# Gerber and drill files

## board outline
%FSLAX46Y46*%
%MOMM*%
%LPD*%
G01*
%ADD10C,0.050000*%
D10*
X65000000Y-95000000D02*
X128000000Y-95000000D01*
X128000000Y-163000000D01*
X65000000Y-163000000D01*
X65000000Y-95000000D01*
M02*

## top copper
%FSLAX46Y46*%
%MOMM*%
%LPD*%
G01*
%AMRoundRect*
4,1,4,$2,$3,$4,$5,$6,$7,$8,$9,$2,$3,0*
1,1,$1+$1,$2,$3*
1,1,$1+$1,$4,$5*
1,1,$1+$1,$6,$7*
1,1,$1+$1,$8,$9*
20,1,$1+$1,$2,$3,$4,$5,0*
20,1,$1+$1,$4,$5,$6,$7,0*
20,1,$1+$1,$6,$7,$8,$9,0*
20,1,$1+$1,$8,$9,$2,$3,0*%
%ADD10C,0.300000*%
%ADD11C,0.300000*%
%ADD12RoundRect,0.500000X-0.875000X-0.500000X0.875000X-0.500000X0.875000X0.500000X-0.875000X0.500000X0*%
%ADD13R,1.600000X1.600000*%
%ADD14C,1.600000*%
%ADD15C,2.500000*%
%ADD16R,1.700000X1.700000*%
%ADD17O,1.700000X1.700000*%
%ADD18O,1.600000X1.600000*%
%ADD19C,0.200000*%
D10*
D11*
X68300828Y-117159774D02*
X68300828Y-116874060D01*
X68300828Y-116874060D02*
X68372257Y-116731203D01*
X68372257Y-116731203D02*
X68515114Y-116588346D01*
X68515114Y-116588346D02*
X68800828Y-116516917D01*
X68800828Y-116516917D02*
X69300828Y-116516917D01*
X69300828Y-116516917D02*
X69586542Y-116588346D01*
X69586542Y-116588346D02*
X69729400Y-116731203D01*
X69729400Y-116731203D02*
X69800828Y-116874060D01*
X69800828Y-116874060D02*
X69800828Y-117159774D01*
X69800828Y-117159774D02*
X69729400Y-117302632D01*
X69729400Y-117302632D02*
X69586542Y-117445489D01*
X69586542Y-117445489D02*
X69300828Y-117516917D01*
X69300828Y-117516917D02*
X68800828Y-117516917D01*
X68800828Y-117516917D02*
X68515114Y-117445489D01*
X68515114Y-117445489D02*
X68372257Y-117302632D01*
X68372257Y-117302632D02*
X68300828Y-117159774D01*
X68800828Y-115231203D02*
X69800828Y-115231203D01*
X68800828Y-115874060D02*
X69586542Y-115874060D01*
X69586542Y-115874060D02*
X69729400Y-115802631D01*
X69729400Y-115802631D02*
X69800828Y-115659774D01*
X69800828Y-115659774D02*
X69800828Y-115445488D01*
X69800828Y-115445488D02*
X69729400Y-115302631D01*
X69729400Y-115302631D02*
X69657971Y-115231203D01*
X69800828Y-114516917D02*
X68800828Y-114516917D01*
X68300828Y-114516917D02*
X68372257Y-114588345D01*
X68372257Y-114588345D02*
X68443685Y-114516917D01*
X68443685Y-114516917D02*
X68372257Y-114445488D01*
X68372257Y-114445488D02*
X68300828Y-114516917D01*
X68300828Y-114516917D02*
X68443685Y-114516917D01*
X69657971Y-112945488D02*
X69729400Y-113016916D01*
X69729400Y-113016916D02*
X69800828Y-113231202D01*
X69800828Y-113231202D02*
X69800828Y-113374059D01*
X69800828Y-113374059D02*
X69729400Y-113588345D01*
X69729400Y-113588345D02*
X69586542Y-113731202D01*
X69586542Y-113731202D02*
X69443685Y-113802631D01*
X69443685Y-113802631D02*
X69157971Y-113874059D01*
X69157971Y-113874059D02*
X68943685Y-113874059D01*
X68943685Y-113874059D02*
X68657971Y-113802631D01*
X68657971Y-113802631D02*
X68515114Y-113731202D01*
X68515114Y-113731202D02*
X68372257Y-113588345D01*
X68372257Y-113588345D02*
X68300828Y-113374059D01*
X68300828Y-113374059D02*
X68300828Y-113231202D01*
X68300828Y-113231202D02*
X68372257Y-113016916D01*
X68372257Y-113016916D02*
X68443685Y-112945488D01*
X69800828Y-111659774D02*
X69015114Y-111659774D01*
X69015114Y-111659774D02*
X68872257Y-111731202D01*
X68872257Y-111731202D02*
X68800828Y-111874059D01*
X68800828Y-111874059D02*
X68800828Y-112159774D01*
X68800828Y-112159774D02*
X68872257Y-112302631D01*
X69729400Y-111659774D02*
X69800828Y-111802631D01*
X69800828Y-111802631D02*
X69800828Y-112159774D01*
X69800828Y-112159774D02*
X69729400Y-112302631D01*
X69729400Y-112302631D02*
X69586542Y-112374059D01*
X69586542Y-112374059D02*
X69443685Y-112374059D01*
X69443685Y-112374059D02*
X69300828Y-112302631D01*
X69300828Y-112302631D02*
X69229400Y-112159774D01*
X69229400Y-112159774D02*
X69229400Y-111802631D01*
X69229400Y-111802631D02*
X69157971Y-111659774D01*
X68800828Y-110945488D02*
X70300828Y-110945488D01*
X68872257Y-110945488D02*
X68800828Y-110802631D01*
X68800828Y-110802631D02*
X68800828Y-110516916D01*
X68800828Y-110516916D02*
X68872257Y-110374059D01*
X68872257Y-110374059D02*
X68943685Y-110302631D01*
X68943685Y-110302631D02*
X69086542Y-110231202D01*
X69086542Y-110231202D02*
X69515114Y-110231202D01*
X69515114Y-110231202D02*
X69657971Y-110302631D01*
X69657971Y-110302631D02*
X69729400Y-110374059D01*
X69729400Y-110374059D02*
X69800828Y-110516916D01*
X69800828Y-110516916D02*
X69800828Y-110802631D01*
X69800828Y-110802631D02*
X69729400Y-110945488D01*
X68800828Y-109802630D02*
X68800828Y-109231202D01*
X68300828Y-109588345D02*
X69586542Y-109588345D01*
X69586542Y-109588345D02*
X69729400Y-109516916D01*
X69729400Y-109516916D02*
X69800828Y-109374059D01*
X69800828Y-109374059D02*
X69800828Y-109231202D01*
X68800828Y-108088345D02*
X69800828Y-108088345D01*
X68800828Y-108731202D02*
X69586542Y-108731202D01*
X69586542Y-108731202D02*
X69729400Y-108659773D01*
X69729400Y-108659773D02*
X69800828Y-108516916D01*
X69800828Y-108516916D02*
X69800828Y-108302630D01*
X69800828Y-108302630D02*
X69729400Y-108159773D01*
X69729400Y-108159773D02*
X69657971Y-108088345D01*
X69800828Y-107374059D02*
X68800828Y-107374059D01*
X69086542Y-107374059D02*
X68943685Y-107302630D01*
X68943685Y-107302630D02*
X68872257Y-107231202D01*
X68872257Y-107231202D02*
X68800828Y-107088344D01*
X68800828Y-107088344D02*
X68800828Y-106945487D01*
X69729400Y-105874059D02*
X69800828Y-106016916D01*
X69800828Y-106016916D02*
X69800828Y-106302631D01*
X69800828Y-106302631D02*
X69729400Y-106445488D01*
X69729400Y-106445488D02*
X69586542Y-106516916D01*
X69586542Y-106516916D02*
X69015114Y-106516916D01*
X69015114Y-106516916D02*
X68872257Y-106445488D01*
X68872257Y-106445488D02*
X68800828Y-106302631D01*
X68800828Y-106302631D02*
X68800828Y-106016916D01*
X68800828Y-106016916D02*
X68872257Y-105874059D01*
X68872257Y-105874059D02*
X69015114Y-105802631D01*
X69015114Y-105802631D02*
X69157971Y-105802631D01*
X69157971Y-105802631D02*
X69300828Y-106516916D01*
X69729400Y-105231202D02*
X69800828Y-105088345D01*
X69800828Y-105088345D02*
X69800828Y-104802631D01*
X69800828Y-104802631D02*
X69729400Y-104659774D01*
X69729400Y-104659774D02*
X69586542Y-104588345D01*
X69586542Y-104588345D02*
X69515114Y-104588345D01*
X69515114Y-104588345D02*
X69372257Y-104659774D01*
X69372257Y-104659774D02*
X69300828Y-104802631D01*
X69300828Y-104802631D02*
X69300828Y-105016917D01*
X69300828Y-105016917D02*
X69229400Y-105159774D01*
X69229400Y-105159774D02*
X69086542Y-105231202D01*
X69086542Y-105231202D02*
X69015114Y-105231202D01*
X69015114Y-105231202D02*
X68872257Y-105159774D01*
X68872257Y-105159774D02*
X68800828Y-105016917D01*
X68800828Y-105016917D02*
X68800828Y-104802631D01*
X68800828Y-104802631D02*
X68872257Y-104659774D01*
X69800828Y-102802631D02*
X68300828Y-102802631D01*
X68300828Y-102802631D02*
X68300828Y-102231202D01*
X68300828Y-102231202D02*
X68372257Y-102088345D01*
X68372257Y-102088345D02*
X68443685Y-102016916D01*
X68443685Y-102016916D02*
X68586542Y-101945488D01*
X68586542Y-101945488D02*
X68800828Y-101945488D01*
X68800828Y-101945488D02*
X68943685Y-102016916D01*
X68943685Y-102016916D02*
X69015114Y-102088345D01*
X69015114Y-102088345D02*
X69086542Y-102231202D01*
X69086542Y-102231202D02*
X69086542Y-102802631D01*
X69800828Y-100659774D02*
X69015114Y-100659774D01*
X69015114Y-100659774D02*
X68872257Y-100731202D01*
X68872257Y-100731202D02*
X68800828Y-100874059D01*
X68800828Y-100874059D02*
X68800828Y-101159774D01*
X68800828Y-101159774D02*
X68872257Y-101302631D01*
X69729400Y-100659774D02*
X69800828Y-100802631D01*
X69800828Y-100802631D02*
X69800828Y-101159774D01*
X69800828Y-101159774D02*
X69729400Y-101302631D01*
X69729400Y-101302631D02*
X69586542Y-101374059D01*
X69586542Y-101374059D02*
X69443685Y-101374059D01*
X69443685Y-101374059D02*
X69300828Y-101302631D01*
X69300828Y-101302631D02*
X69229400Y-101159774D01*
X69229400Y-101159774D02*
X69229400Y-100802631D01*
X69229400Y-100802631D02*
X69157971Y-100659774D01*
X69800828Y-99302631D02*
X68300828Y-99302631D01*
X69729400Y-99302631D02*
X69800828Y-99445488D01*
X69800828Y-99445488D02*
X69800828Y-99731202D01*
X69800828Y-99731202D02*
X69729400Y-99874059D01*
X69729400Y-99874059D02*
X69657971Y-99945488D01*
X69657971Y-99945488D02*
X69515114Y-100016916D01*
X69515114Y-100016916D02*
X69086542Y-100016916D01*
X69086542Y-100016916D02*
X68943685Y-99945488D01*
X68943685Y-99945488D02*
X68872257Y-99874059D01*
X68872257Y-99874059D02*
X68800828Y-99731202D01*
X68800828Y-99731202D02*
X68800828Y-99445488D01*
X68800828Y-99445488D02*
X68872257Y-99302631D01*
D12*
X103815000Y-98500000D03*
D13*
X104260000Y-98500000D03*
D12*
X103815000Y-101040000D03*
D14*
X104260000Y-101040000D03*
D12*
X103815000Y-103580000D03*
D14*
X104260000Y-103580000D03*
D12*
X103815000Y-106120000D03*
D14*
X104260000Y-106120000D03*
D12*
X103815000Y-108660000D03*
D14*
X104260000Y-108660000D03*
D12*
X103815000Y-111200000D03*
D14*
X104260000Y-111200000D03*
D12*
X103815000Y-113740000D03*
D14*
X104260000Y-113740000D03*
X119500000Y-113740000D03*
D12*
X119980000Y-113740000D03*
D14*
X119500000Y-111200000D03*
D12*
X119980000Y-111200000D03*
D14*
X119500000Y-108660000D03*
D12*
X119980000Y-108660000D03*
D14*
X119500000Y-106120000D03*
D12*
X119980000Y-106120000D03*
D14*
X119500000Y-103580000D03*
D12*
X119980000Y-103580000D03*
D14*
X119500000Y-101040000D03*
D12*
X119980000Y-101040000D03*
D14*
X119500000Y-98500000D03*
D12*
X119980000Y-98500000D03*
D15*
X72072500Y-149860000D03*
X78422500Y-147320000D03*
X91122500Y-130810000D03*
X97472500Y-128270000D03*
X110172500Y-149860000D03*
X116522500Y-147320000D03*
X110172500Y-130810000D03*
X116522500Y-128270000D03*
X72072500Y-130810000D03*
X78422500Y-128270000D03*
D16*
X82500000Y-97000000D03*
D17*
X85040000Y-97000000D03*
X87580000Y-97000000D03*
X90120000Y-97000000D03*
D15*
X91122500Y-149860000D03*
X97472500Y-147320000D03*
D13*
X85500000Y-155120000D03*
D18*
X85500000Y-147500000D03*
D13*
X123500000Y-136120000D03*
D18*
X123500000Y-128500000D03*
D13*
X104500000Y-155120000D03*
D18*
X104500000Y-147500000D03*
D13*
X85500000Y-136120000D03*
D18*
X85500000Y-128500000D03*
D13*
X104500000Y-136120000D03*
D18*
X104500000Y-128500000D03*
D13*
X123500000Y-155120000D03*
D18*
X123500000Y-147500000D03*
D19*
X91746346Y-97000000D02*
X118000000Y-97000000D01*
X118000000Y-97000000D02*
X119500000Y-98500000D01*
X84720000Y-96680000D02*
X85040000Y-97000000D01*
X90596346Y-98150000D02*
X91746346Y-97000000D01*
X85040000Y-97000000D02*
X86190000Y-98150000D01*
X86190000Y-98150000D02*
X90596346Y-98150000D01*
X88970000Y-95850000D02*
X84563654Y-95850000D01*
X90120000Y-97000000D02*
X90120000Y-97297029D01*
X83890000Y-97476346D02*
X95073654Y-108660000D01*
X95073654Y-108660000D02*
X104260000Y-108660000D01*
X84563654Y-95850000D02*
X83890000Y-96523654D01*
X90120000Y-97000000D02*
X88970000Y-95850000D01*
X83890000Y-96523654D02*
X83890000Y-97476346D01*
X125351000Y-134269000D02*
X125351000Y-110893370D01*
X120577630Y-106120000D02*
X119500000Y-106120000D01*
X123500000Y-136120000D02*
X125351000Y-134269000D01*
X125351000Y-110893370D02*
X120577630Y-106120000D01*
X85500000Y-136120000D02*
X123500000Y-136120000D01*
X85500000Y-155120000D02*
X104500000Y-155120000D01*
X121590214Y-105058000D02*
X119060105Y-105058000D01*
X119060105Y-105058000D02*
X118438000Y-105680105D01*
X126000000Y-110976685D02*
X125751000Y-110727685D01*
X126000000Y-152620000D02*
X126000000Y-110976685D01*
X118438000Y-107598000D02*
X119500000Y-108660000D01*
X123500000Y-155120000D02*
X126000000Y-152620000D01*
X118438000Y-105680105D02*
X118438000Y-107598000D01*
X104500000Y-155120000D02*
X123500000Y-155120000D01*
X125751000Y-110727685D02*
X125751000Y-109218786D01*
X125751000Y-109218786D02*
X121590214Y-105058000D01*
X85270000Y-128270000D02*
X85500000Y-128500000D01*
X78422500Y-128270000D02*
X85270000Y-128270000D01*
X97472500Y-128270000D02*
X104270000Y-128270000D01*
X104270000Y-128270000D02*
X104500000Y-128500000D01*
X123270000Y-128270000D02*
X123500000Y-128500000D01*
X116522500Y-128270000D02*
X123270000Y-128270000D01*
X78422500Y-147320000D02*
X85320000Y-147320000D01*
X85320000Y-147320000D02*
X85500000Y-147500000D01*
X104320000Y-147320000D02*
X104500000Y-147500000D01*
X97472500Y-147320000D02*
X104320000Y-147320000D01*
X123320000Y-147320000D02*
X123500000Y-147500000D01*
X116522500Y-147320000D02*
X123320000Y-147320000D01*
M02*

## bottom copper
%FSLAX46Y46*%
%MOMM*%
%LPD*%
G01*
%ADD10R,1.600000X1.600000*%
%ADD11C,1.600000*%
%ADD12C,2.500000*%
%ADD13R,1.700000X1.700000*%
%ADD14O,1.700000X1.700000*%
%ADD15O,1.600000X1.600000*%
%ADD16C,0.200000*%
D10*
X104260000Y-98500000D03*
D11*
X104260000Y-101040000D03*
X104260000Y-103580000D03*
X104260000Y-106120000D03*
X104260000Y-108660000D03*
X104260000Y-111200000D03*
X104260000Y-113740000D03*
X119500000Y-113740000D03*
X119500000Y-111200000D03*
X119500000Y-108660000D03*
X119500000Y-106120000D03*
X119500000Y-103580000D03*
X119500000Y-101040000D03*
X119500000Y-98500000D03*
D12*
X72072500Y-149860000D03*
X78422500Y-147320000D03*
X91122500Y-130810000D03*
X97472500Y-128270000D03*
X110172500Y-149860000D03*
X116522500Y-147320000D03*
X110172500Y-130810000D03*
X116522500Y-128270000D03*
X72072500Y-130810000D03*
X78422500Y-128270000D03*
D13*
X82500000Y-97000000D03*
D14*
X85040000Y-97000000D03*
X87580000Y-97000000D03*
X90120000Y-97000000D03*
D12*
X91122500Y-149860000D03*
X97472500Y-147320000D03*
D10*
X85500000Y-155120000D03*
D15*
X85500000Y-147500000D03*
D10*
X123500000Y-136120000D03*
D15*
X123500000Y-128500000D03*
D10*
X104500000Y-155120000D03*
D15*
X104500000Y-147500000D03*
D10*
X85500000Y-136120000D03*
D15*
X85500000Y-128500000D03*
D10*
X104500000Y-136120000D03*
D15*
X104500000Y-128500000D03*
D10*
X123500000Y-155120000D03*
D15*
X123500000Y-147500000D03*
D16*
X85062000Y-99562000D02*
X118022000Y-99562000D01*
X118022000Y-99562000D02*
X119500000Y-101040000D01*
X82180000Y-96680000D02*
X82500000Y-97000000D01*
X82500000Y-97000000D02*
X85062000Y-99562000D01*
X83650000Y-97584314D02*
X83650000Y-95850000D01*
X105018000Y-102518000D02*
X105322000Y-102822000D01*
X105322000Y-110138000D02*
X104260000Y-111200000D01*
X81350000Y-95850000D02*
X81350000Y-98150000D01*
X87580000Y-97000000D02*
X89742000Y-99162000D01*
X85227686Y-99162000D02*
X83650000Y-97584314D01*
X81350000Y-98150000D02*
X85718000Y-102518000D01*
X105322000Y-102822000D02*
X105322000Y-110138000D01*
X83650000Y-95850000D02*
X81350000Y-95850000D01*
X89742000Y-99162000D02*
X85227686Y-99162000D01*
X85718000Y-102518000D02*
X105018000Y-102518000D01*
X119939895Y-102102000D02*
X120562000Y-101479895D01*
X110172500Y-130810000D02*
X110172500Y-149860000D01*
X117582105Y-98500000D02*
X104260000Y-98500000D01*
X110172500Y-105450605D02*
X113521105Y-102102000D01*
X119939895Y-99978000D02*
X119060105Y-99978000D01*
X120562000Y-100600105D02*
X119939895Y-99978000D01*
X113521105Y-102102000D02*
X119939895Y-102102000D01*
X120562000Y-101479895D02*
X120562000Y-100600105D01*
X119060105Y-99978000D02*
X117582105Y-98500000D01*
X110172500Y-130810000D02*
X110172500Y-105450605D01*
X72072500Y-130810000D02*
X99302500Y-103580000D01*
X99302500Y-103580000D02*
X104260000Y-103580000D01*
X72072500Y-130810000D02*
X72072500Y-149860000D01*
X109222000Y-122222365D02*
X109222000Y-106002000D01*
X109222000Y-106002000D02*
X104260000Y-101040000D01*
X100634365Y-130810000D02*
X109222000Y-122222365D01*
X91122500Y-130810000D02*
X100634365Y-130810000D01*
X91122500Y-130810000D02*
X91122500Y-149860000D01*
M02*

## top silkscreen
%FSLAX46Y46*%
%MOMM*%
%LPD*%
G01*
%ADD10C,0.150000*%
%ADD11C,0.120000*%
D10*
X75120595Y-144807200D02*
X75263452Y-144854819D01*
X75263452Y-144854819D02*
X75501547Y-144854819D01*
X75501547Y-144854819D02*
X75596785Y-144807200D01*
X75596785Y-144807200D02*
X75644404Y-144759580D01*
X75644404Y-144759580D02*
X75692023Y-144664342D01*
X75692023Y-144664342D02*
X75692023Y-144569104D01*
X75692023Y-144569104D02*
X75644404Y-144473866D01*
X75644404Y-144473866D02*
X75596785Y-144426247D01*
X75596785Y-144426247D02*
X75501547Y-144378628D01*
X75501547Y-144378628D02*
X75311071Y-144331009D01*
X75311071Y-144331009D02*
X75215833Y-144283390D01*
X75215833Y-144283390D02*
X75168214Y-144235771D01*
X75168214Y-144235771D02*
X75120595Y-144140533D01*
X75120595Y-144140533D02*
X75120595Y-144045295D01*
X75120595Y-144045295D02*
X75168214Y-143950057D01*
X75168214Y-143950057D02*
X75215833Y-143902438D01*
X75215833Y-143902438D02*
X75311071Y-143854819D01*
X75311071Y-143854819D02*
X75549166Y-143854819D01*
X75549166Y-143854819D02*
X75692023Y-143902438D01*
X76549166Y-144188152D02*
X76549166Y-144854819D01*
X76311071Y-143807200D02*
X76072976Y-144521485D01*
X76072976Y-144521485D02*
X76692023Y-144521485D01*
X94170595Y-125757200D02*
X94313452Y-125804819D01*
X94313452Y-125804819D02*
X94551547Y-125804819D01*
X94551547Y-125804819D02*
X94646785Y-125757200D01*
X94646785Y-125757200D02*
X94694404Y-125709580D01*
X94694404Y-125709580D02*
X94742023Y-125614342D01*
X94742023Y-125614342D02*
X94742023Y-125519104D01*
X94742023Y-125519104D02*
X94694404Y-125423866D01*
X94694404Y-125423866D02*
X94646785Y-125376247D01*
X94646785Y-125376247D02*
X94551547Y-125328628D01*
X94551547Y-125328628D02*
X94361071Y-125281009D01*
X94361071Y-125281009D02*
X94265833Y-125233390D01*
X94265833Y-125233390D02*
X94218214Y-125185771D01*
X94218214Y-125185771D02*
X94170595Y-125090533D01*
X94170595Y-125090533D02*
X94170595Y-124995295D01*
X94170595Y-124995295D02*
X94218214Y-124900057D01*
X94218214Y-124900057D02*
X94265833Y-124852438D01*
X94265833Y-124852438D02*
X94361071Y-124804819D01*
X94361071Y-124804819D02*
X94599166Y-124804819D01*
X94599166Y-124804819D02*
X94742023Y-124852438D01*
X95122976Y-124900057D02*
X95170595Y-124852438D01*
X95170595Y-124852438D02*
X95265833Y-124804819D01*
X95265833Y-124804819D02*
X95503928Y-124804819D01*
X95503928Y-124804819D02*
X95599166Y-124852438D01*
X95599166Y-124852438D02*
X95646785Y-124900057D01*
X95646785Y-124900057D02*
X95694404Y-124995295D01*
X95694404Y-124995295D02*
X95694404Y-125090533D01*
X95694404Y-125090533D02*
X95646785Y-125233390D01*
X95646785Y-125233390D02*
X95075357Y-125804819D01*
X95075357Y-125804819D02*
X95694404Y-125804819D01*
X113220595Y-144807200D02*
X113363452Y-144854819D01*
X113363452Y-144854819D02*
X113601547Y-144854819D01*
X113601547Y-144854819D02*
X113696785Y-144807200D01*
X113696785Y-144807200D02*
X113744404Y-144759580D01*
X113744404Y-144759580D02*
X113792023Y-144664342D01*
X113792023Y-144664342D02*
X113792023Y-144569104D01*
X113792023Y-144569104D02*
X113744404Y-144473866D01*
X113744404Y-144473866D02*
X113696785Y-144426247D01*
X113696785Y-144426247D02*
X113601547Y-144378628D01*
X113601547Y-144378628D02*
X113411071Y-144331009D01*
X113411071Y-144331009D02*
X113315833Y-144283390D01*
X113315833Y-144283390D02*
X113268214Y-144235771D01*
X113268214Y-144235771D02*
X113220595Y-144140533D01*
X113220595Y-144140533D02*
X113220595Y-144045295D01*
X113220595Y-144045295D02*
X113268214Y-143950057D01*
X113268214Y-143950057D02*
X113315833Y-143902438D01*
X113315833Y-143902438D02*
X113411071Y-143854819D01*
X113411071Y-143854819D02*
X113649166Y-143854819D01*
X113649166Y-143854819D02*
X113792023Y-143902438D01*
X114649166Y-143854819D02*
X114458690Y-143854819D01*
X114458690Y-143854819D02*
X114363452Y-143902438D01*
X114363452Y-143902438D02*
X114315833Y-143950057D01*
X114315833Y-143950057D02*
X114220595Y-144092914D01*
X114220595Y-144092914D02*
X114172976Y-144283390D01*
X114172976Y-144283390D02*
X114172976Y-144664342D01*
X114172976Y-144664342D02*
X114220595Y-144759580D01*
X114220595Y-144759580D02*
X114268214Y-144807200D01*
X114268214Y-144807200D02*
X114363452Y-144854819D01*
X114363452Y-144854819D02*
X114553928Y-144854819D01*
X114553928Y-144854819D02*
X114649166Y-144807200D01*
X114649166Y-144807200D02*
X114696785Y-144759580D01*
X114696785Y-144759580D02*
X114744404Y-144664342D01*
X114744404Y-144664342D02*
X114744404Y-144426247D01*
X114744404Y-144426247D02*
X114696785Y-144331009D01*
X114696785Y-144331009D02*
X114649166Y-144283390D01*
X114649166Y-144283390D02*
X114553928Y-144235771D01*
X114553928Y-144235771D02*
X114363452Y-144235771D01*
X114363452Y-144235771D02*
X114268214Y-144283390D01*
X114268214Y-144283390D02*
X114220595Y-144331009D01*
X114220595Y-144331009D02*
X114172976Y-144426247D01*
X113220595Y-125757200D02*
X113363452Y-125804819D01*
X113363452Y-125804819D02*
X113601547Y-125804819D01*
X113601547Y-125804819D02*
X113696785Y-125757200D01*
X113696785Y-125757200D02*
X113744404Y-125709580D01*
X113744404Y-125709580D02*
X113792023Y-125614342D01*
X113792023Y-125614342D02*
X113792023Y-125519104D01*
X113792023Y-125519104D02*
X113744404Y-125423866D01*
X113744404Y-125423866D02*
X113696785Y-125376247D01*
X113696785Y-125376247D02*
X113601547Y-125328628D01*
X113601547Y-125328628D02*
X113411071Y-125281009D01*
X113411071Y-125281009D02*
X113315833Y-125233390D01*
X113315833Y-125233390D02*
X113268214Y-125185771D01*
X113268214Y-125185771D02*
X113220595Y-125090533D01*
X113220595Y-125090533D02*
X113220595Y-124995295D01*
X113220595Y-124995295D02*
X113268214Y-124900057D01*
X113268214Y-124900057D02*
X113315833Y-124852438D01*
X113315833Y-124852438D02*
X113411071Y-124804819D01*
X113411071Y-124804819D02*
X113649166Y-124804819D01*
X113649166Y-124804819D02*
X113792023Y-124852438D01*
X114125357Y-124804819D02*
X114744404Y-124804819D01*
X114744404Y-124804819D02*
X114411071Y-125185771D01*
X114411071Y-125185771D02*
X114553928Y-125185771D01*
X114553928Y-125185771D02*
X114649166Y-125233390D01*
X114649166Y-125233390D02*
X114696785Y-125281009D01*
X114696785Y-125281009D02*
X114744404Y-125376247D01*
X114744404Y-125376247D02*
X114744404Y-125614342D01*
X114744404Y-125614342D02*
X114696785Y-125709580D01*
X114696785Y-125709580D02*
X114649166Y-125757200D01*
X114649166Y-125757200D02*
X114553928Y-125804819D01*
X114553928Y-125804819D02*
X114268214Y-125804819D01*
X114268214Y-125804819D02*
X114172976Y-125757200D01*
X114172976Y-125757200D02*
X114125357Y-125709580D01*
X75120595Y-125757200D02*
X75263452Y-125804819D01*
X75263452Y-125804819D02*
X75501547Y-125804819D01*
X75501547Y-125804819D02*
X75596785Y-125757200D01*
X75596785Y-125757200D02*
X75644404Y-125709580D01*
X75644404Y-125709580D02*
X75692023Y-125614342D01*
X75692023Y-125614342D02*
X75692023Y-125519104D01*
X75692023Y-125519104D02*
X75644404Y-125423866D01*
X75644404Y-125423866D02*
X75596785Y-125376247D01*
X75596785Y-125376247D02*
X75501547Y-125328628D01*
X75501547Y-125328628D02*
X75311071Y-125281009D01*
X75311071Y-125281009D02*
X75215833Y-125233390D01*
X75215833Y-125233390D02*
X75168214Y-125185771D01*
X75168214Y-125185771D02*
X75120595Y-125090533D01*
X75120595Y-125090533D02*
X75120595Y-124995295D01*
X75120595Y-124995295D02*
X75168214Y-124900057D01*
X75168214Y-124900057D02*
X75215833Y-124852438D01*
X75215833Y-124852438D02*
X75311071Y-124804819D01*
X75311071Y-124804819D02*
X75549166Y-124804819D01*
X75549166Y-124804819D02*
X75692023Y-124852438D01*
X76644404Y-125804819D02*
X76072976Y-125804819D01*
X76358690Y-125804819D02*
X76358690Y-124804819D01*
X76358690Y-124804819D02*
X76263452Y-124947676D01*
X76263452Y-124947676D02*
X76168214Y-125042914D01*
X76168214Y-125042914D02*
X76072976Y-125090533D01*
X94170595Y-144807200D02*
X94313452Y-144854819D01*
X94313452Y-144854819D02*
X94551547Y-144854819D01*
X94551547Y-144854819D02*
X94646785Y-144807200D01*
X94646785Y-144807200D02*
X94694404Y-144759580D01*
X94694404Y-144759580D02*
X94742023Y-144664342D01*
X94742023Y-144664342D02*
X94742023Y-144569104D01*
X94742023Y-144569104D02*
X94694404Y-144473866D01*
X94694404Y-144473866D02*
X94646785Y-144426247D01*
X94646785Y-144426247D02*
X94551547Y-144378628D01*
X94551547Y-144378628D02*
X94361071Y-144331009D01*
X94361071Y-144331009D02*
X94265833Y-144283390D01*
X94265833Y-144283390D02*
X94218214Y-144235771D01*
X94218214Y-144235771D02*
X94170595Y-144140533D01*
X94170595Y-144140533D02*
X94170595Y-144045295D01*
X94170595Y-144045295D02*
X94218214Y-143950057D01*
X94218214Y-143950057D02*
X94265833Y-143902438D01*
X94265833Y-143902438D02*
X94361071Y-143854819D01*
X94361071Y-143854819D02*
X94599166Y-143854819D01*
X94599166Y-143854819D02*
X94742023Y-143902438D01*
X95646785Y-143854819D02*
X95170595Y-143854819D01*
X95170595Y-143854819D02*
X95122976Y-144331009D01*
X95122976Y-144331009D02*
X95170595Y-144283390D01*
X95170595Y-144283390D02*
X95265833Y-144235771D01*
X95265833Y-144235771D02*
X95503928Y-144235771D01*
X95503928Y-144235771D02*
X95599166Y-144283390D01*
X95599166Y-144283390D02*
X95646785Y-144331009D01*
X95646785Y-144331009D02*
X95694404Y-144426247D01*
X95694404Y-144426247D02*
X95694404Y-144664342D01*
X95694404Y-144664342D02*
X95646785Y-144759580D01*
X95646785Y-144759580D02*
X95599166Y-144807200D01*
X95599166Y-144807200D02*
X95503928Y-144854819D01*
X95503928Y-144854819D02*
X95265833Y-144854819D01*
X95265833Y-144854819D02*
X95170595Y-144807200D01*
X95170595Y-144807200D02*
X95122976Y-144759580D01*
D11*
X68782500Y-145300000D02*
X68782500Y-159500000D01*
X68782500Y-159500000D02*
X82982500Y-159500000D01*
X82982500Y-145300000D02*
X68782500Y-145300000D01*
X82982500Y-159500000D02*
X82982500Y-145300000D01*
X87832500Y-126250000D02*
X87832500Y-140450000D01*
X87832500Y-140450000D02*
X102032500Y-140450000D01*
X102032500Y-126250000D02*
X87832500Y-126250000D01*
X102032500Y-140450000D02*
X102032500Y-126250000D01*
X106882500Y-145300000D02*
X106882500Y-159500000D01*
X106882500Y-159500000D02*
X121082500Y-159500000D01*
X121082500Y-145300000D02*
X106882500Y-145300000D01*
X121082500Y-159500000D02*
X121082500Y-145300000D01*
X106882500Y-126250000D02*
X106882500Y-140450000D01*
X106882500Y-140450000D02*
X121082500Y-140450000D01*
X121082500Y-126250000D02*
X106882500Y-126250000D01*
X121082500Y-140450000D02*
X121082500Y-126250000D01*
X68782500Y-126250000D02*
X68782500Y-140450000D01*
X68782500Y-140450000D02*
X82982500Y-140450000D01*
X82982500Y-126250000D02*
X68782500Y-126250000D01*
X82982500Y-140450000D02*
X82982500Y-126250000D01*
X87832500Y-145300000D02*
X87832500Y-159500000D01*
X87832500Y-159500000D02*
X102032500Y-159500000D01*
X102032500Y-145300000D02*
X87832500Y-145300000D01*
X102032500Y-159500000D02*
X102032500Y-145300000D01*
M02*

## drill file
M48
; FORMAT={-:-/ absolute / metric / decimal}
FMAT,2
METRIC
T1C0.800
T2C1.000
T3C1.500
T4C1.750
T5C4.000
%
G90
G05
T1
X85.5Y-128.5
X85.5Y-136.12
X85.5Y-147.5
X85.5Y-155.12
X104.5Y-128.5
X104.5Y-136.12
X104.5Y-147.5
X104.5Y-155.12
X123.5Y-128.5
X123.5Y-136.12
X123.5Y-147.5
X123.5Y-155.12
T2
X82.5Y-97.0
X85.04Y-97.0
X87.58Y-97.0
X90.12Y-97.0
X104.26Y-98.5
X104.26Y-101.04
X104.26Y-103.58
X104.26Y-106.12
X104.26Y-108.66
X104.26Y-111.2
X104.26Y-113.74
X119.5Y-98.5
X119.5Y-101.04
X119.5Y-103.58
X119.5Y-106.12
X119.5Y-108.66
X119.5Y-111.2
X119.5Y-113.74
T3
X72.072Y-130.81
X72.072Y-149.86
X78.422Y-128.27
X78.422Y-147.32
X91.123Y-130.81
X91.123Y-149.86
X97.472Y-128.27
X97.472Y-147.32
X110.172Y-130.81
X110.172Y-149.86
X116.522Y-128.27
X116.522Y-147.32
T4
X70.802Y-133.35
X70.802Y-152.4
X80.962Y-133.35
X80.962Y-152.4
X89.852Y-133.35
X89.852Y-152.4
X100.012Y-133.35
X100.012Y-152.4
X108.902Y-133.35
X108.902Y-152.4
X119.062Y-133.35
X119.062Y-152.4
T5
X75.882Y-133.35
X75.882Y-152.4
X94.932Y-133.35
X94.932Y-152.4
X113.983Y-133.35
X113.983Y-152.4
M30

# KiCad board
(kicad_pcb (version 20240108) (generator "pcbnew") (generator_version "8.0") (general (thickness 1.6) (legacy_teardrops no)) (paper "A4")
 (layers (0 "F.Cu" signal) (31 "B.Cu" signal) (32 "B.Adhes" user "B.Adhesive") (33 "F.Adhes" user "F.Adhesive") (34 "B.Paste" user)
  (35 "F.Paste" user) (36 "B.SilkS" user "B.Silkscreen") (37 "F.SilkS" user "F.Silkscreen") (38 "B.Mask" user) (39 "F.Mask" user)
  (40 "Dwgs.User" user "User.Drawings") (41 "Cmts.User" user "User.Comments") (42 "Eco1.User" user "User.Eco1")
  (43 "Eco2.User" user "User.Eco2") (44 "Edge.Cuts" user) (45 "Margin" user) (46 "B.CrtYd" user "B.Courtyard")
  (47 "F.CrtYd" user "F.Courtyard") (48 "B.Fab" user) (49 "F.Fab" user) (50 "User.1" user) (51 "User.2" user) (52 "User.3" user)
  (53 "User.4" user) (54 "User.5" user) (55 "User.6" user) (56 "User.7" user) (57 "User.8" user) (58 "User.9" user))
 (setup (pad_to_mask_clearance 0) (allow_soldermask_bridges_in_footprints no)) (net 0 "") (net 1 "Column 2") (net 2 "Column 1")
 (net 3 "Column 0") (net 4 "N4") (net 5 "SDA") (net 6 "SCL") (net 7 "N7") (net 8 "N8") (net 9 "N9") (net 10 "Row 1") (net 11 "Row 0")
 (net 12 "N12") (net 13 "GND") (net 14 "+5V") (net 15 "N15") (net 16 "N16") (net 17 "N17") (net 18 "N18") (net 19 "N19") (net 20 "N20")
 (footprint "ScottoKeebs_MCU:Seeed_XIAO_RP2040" (layer "F.Cu") (at 111.88 106.12)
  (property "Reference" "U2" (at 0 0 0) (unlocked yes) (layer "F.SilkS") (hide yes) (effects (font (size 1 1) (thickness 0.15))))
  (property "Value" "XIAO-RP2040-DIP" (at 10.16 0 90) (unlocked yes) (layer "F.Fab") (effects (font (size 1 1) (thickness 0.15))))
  (pad "1" smd roundrect (at -8.065 -7.62) (size 2.75 2) (layers "F.Cu" "F.Paste" "F.Mask") (roundrect_rratio 0.25) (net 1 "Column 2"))
  (pad "1" thru_hole rect (at -7.62 -7.62 90) (size 1.6 1.6) (drill 1) (layers "*.Cu" "*.Mask") (remove_unused_layers no) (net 1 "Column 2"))
  (pad "2" smd roundrect (at -8.065 -5.08) (size 2.75 2) (layers "F.Cu" "F.Paste" "F.Mask") (roundrect_rratio 0.25) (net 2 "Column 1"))
  (pad "2" thru_hole circle (at -7.62 -5.08 90) (size 1.6 1.6) (drill 1) (layers "*.Cu" "*.Mask") (remove_unused_layers no)
   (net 2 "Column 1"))
  (pad "3" smd roundrect (at -8.065 -2.54) (size 2.75 2) (layers "F.Cu" "F.Paste" "F.Mask") (roundrect_rratio 0.25) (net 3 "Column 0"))
  (pad "3" thru_hole circle (at -7.62 -2.54 90) (size 1.6 1.6) (drill 1) (layers "*.Cu" "*.Mask") (remove_unused_layers no)
   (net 3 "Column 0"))
  (pad "4" smd roundrect (at -8.065 0) (size 2.75 2) (layers "F.Cu" "F.Paste" "F.Mask") (roundrect_rratio 0.25) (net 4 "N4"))
  (pad "4" thru_hole circle (at -7.62 0 90) (size 1.6 1.6) (drill 1) (layers "*.Cu" "*.Mask") (remove_unused_layers no) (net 4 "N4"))
  (pad "5" smd roundrect (at -8.065 2.54) (size 2.75 2) (layers "F.Cu" "F.Paste" "F.Mask") (roundrect_rratio 0.25) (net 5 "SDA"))
  (pad "5" thru_hole circle (at -7.62 2.54 90) (size 1.6 1.6) (drill 1) (layers "*.Cu" "*.Mask") (remove_unused_layers no) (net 5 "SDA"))
  (pad "6" smd roundrect (at -8.065 5.08) (size 2.75 2) (layers "F.Cu" "F.Paste" "F.Mask") (roundrect_rratio 0.25) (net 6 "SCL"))
  (pad "6" thru_hole circle (at -7.62 5.08 90) (size 1.6 1.6) (drill 1) (layers "*.Cu" "*.Mask") (remove_unused_layers no) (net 6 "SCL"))
  (pad "7" smd roundrect (at -8.065 7.62) (size 2.75 2) (layers "F.Cu" "F.Paste" "F.Mask") (roundrect_rratio 0.25) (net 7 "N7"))
  (pad "7" thru_hole circle (at -7.62 7.62 90) (size 1.6 1.6) (drill 1) (layers "*.Cu" "*.Mask") (remove_unused_layers no) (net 7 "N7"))
  (pad "8" thru_hole circle (at 7.62 7.62 90) (size 1.6 1.6) (drill 1) (layers "*.Cu" "*.Mask") (remove_unused_layers no) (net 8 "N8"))
  (pad "8" smd roundrect (at 8.1 7.62) (size 2.75 2) (layers "F.Cu" "F.Paste" "F.Mask") (roundrect_rratio 0.25) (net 8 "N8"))
  (pad "9" thru_hole circle (at 7.62 5.08 90) (size 1.6 1.6) (drill 1) (layers "*.Cu" "*.Mask") (remove_unused_layers no) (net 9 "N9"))
  (pad "9" smd roundrect (at 8.1 5.08) (size 2.75 2) (layers "F.Cu" "F.Paste" "F.Mask") (roundrect_rratio 0.25) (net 9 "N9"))
  (pad "10" thru_hole circle (at 7.62 2.54 90) (size 1.6 1.6) (drill 1) (layers "*.Cu" "*.Mask") (remove_unused_layers no) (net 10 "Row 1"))
  (pad "10" smd roundrect (at 8.1 2.54) (size 2.75 2) (layers "F.Cu" "F.Paste" "F.Mask") (roundrect_rratio 0.25) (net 10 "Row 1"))
  (pad "11" thru_hole circle (at 7.62 0 90) (size 1.6 1.6) (drill 1) (layers "*.Cu" "*.Mask") (remove_unused_layers no) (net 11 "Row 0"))
  (pad "11" smd roundrect (at 8.1 0) (size 2.75 2) (layers "F.Cu" "F.Paste" "F.Mask") (roundrect_rratio 0.25) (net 11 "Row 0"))
  (pad "12" thru_hole circle (at 7.62 -2.54 90) (size 1.6 1.6) (drill 1) (layers "*.Cu" "*.Mask") (remove_unused_layers no) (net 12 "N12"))
  (pad "12" smd roundrect (at 8.1 -2.54) (size 2.75 2) (layers "F.Cu" "F.Paste" "F.Mask") (roundrect_rratio 0.25) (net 12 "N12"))
  (pad "13" thru_hole circle (at 7.62 -5.08 90) (size 1.6 1.6) (drill 1) (layers "*.Cu" "*.Mask") (remove_unused_layers no) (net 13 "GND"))
  (pad "13" smd roundrect (at 8.1 -5.08) (size 2.75 2) (layers "F.Cu" "F.Paste" "F.Mask") (roundrect_rratio 0.25) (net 13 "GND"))
  (pad "14" thru_hole circle (at 7.62 -7.62 90) (size 1.6 1.6) (drill 1) (layers "*.Cu" "*.Mask") (remove_unused_layers no) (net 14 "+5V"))
  (pad "14" smd roundrect (at 8.1 -7.62) (size 2.75 2) (layers "F.Cu" "F.Paste" "F.Mask") (roundrect_rratio 0.25) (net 14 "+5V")))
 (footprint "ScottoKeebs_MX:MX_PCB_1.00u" (layer "F.Cu") (at 75.8825 152.4)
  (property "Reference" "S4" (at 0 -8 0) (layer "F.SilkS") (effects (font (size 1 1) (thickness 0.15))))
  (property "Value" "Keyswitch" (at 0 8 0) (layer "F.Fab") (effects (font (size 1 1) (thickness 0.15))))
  (fp_line (start -7.1 -7.1) (end -7.1 7.1) (stroke (width 0.12) (type solid)) (layer "F.SilkS"))
  (fp_line (start -7.1 7.1) (end 7.1 7.1) (stroke (width 0.12) (type solid)) (layer "F.SilkS"))
  (fp_line (start 7.1 -7.1) (end -7.1 -7.1) (stroke (width 0.12) (type solid)) (layer "F.SilkS"))
  (fp_line (start 7.1 7.1) (end 7.1 -7.1) (stroke (width 0.12) (type solid)) (layer "F.SilkS"))
  (pad "" np_thru_hole circle (at -5.08 0) (size 1.75 1.75) (drill 1.75) (layers "*.Cu" "*.Mask"))
  (pad "" np_thru_hole circle (at 0 0) (size 4 4) (drill 4) (layers "*.Cu" "*.Mask"))
  (pad "" np_thru_hole circle (at 5.08 0) (size 1.75 1.75) (drill 1.75) (layers "*.Cu" "*.Mask"))
  (pad "1" thru_hole circle (at -3.81 -2.54) (size 2.5 2.5) (drill 1.5) (layers "*.Cu" "*.Mask") (remove_unused_layers no)
   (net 3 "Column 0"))
  (pad "2" thru_hole circle (at 2.54 -5.08) (size 2.5 2.5) (drill 1.5) (layers "*.Cu" "*.Mask") (remove_unused_layers no) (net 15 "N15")))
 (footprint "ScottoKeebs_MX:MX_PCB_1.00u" (layer "F.Cu") (at 94.9325 133.35)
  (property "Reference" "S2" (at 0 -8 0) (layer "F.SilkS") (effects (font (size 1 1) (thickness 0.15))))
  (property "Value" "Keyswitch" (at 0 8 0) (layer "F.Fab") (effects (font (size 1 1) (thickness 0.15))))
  (fp_line (start -7.1 -7.1) (end -7.1 7.1) (stroke (width 0.12) (type solid)) (layer "F.SilkS"))
  (fp_line (start -7.1 7.1) (end 7.1 7.1) (stroke (width 0.12) (type solid)) (layer "F.SilkS"))
  (fp_line (start 7.1 -7.1) (end -7.1 -7.1) (stroke (width 0.12) (type solid)) (layer "F.SilkS"))
  (fp_line (start 7.1 7.1) (end 7.1 -7.1) (stroke (width 0.12) (type solid)) (layer "F.SilkS"))
  (pad "" np_thru_hole circle (at -5.08 0) (size 1.75 1.75) (drill 1.75) (layers "*.Cu" "*.Mask"))
  (pad "" np_thru_hole circle (at 0 0) (size 4 4) (drill 4) (layers "*.Cu" "*.Mask"))
  (pad "" np_thru_hole circle (at 5.08 0) (size 1.75 1.75) (drill 1.75) (layers "*.Cu" "*.Mask"))
  (pad "1" thru_hole circle (at -3.81 -2.54) (size 2.5 2.5) (drill 1.5) (layers "*.Cu" "*.Mask") (remove_unused_layers no)
   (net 2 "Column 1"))
  (pad "2" thru_hole circle (at 2.54 -5.08) (size 2.5 2.5) (drill 1.5) (layers "*.Cu" "*.Mask") (remove_unused_layers no) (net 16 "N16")))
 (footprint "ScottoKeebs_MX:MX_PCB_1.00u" (layer "F.Cu") (at 113.9825 152.4)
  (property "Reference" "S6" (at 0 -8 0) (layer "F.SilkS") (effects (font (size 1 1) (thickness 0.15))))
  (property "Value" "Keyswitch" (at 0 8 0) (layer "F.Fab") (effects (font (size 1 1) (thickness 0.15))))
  (fp_line (start -7.1 -7.1) (end -7.1 7.1) (stroke (width 0.12) (type solid)) (layer "F.SilkS"))
  (fp_line (start -7.1 7.1) (end 7.1 7.1) (stroke (width 0.12) (type solid)) (layer "F.SilkS"))
  (fp_line (start 7.1 -7.1) (end -7.1 -7.1) (stroke (width 0.12) (type solid)) (layer "F.SilkS"))
  (fp_line (start 7.1 7.1) (end 7.1 -7.1) (stroke (width 0.12) (type solid)) (layer "F.SilkS"))
  (pad "" np_thru_hole circle (at -5.08 0) (size 1.75 1.75) (drill 1.75) (layers "*.Cu" "*.Mask"))
  (pad "" np_thru_hole circle (at 0 0) (size 4 4) (drill 4) (layers "*.Cu" "*.Mask"))
  (pad "" np_thru_hole circle (at 5.08 0) (size 1.75 1.75) (drill 1.75) (layers "*.Cu" "*.Mask"))
  (pad "1" thru_hole circle (at -3.81 -2.54) (size 2.5 2.5) (drill 1.5) (layers "*.Cu" "*.Mask") (remove_unused_layers no)
   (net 1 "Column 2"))
  (pad "2" thru_hole circle (at 2.54 -5.08) (size 2.5 2.5) (drill 1.5) (layers "*.Cu" "*.Mask") (remove_unused_layers no) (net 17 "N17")))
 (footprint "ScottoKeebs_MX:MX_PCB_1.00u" (layer "F.Cu") (at 113.9825 133.35)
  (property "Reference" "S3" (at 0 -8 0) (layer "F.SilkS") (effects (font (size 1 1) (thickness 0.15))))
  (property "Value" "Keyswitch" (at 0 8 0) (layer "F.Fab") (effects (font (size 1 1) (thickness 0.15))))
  (fp_line (start -7.1 -7.1) (end -7.1 7.1) (stroke (width 0.12) (type solid)) (layer "F.SilkS"))
  (fp_line (start -7.1 7.1) (end 7.1 7.1) (stroke (width 0.12) (type solid)) (layer "F.SilkS"))
  (fp_line (start 7.1 -7.1) (end -7.1 -7.1) (stroke (width 0.12) (type solid)) (layer "F.SilkS"))
  (fp_line (start 7.1 7.1) (end 7.1 -7.1) (stroke (width 0.12) (type solid)) (layer "F.SilkS"))
  (pad "" np_thru_hole circle (at -5.08 0) (size 1.75 1.75) (drill 1.75) (layers "*.Cu" "*.Mask"))
  (pad "" np_thru_hole circle (at 0 0) (size 4 4) (drill 4) (layers "*.Cu" "*.Mask"))
  (pad "" np_thru_hole circle (at 5.08 0) (size 1.75 1.75) (drill 1.75) (layers "*.Cu" "*.Mask"))
  (pad "1" thru_hole circle (at -3.81 -2.54) (size 2.5 2.5) (drill 1.5) (layers "*.Cu" "*.Mask") (remove_unused_layers no)
   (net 1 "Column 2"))
  (pad "2" thru_hole circle (at 2.54 -5.08) (size 2.5 2.5) (drill 1.5) (layers "*.Cu" "*.Mask") (remove_unused_layers no) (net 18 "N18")))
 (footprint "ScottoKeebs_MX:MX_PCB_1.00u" (layer "F.Cu") (at 75.8825 133.35)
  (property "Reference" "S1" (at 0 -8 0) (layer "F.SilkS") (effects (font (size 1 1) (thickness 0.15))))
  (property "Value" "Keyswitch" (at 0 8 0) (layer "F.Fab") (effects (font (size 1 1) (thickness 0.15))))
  (fp_line (start -7.1 -7.1) (end -7.1 7.1) (stroke (width 0.12) (type solid)) (layer "F.SilkS"))
  (fp_line (start -7.1 7.1) (end 7.1 7.1) (stroke (width 0.12) (type solid)) (layer "F.SilkS"))
  (fp_line (start 7.1 -7.1) (end -7.1 -7.1) (stroke (width 0.12) (type solid)) (layer "F.SilkS"))
  (fp_line (start 7.1 7.1) (end 7.1 -7.1) (stroke (width 0.12) (type solid)) (layer "F.SilkS"))
  (pad "" np_thru_hole circle (at -5.08 0) (size 1.75 1.75) (drill 1.75) (layers "*.Cu" "*.Mask"))
  (pad "" np_thru_hole circle (at 0 0) (size 4 4) (drill 4) (layers "*.Cu" "*.Mask"))
  (pad "" np_thru_hole circle (at 5.08 0) (size 1.75 1.75) (drill 1.75) (layers "*.Cu" "*.Mask"))
  (pad "1" thru_hole circle (at -3.81 -2.54) (size 2.5 2.5) (drill 1.5) (layers "*.Cu" "*.Mask") (remove_unused_layers no)
   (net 3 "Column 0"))
  (pad "2" thru_hole circle (at 2.54 -5.08) (size 2.5 2.5) (drill 1.5) (layers "*.Cu" "*.Mask") (remove_unused_layers no) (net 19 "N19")))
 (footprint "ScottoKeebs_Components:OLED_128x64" (layer "F.Cu") (at 86.31 97)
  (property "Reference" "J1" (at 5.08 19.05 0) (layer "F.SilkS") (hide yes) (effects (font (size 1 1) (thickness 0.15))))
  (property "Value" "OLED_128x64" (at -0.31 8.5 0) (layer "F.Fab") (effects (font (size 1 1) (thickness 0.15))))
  (pad "1" thru_hole rect (at -3.81 0 90) (size 1.7 1.7) (drill 1) (layers "*.Cu" "*.Mask") (remove_unused_layers no) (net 13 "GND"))
  (pad "2" thru_hole oval (at -1.27 0 90) (size 1.7 1.7) (drill 1) (layers "*.Cu" "*.Mask") (remove_unused_layers no) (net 14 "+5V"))
  (pad "3" thru_hole oval (at 1.27 0 90) (size 1.7 1.7) (drill 1) (layers "*.Cu" "*.Mask") (remove_unused_layers no) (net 6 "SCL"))
  (pad "4" thru_hole oval (at 3.81 0 90) (size 1.7 1.7) (drill 1) (layers "*.Cu" "*.Mask") (remove_unused_layers no) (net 5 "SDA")))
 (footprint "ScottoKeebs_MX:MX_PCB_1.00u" (layer "F.Cu") (at 94.9325 152.4)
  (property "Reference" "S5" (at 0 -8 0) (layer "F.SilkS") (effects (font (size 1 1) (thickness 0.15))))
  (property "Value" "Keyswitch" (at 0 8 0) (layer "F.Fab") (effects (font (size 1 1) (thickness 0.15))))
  (fp_line (start -7.1 -7.1) (end -7.1 7.1) (stroke (width 0.12) (type solid)) (layer "F.SilkS"))
  (fp_line (start -7.1 7.1) (end 7.1 7.1) (stroke (width 0.12) (type solid)) (layer "F.SilkS"))
  (fp_line (start 7.1 -7.1) (end -7.1 -7.1) (stroke (width 0.12) (type solid)) (layer "F.SilkS"))
  (fp_line (start 7.1 7.1) (end 7.1 -7.1) (stroke (width 0.12) (type solid)) (layer "F.SilkS"))
  (pad "" np_thru_hole circle (at -5.08 0) (size 1.75 1.75) (drill 1.75) (layers "*.Cu" "*.Mask"))
  (pad "" np_thru_hole circle (at 0 0) (size 4 4) (drill 4) (layers "*.Cu" "*.Mask"))
  (pad "" np_thru_hole circle (at 5.08 0) (size 1.75 1.75) (drill 1.75) (layers "*.Cu" "*.Mask"))
  (pad "1" thru_hole circle (at -3.81 -2.54) (size 2.5 2.5) (drill 1.5) (layers "*.Cu" "*.Mask") (remove_unused_layers no)
   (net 2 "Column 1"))
  (pad "2" thru_hole circle (at 2.54 -5.08) (size 2.5 2.5) (drill 1.5) (layers "*.Cu" "*.Mask") (remove_unused_layers no) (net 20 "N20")))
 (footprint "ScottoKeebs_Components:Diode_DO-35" (layer "B.Cu") (at 85.5 155.12 90)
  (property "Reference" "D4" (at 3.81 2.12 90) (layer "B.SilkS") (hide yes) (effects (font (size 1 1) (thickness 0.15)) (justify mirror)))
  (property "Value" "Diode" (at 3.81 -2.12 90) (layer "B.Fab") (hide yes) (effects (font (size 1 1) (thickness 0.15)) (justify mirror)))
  (pad "1" thru_hole rect (at 0 0 90) (size 1.6 1.6) (drill 0.8) (layers "*.Cu" "*.Mask") (remove_unused_layers no) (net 10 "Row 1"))
  (pad "2" thru_hole oval (at 7.62 0 90) (size 1.6 1.6) (drill 0.8) (layers "*.Cu" "*.Mask") (remove_unused_layers no) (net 15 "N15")))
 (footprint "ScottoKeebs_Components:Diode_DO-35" (layer "B.Cu") (at 123.5 136.12 90)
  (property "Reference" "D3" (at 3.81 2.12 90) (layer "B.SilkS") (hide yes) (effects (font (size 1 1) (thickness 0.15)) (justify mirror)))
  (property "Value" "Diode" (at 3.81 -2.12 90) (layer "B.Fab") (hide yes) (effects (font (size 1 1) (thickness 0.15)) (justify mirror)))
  (pad "1" thru_hole rect (at 0 0 90) (size 1.6 1.6) (drill 0.8) (layers "*.Cu" "*.Mask") (remove_unused_layers no) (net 11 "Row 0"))
  (pad "2" thru_hole oval (at 7.62 0 90) (size 1.6 1.6) (drill 0.8) (layers "*.Cu" "*.Mask") (remove_unused_layers no) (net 18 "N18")))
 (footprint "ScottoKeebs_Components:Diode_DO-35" (layer "B.Cu") (at 104.5 155.12 90)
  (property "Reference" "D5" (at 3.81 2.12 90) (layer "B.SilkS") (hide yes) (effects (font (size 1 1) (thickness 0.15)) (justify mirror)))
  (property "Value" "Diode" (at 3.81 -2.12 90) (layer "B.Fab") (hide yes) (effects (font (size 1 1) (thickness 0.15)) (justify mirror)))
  (pad "1" thru_hole rect (at 0 0 90) (size 1.6 1.6) (drill 0.8) (layers "*.Cu" "*.Mask") (remove_unused_layers no) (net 10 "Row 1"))
  (pad "2" thru_hole oval (at 7.62 0 90) (size 1.6 1.6) (drill 0.8) (layers "*.Cu" "*.Mask") (remove_unused_layers no) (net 20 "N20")))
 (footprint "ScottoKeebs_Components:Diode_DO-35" (layer "B.Cu") (at 85.5 136.12 90)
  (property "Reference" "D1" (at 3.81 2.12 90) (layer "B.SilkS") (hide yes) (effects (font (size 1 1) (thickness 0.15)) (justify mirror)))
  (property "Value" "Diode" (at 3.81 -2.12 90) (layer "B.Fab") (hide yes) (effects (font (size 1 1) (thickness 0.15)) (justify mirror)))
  (pad "1" thru_hole rect (at 0 0 90) (size 1.6 1.6) (drill 0.8) (layers "*.Cu" "*.Mask") (remove_unused_layers no) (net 11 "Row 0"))
  (pad "2" thru_hole oval (at 7.62 0 90) (size 1.6 1.6) (drill 0.8) (layers "*.Cu" "*.Mask") (remove_unused_layers no) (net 19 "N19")))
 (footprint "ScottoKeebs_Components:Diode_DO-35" (layer "B.Cu") (at 104.5 136.12 90)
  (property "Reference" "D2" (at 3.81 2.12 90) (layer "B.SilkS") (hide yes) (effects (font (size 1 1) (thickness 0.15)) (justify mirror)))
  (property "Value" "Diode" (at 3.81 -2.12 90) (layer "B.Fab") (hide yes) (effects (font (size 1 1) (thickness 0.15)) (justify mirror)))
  (pad "1" thru_hole rect (at 0 0 90) (size 1.6 1.6) (drill 0.8) (layers "*.Cu" "*.Mask") (remove_unused_layers no) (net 11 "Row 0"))
  (pad "2" thru_hole oval (at 7.62 0 90) (size 1.6 1.6) (drill 0.8) (layers "*.Cu" "*.Mask") (remove_unused_layers no) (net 16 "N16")))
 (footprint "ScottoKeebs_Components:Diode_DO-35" (layer "B.Cu") (at 123.5 155.12 90)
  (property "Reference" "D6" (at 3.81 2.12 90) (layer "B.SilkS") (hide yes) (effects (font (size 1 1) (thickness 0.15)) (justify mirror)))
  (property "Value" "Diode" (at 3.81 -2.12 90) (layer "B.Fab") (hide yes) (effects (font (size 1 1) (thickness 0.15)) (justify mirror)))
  (pad "1" thru_hole rect (at 0 0 90) (size 1.6 1.6) (drill 0.8) (layers "*.Cu" "*.Mask") (remove_unused_layers no) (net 10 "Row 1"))
  (pad "2" thru_hole oval (at 7.62 0 90) (size 1.6 1.6) (drill 0.8) (layers "*.Cu" "*.Mask") (remove_unused_layers no) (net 17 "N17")))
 (gr_rect (start 65 95) (end 128 163) (stroke (width 0.05) (type default)) (fill none) (layer "Edge.Cuts"))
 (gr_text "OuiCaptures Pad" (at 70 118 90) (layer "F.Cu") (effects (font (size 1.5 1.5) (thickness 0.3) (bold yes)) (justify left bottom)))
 (segment (start 85.062 99.562) (end 118.022 99.562) (width 0.2) (layer "B.Cu") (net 13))
 (segment (start 118.022 99.562) (end 119.5 101.04) (width 0.2) (layer "B.Cu") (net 13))
 (segment (start 82.18 96.68) (end 82.5 97) (width 0.2) (layer "B.Cu") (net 13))
 (segment (start 82.5 97) (end 85.062 99.562) (width 0.2) (layer "B.Cu") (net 13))
 (segment (start 91.746346 97) (end 118 97) (width 0.2) (layer "F.Cu") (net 14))
 (segment (start 118 97) (end 119.5 98.5) (width 0.2) (layer "F.Cu") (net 14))
 (segment (start 84.72 96.68) (end 85.04 97) (width 0.2) (layer "F.Cu") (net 14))
 (segment (start 90.596346 98.15) (end 91.746346 97) (width 0.2) (layer "F.Cu") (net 14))
 (segment (start 85.04 97) (end 86.19 98.15) (width 0.2) (layer "F.Cu") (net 14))
 (segment (start 86.19 98.15) (end 90.596346 98.15) (width 0.2) (layer "F.Cu") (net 14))
 (segment (start 83.65 97.584314) (end 83.65 95.85) (width 0.2) (layer "B.Cu") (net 6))
 (segment (start 105.018 102.518) (end 105.322 102.822) (width 0.2) (layer "B.Cu") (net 6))
 (segment (start 105.322 110.138) (end 104.26 111.2) (width 0.2) (layer "B.Cu") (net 6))
 (segment (start 81.35 95.85) (end 81.35 98.15) (width 0.2) (layer "B.Cu") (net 6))
 (segment (start 87.58 97) (end 89.742 99.162) (width 0.2) (layer "B.Cu") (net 6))
 (segment (start 85.227686 99.162) (end 83.65 97.584314) (width 0.2) (layer "B.Cu") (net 6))
 (segment (start 81.35 98.15) (end 85.718 102.518) (width 0.2) (layer "B.Cu") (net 6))
 (segment (start 105.322 102.822) (end 105.322 110.138) (width 0.2) (layer "B.Cu") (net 6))
 (segment (start 83.65 95.85) (end 81.35 95.85) (width 0.2) (layer "B.Cu") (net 6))
 (segment (start 89.742 99.162) (end 85.227686 99.162) (width 0.2) (layer "B.Cu") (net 6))
 (segment (start 85.718 102.518) (end 105.018 102.518) (width 0.2) (layer "B.Cu") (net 6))
 (segment (start 88.97 95.85) (end 84.563654 95.85) (width 0.2) (layer "F.Cu") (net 5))
 (segment (start 90.12 97) (end 90.12 97.297029) (width 0.2) (layer "F.Cu") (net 5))
 (segment (start 83.89 97.476346) (end 95.073654 108.66) (width 0.2) (layer "F.Cu") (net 5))
 (segment (start 95.073654 108.66) (end 104.26 108.66) (width 0.2) (layer "F.Cu") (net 5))
 (segment (start 84.563654 95.85) (end 83.89 96.523654) (width 0.2) (layer "F.Cu") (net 5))
 (segment (start 90.12 97) (end 88.97 95.85) (width 0.2) (layer "F.Cu") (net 5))
 (segment (start 83.89 96.523654) (end 83.89 97.476346) (width 0.2) (layer "F.Cu") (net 5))
 (segment (start 119.939895 102.102) (end 120.562 101.479895) (width 0.2) (layer "B.Cu") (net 1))
 (segment (start 110.1725 130.81) (end 110.1725 149.86) (width 0.2) (layer "B.Cu") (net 1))
 (segment (start 117.582105 98.5) (end 104.26 98.5) (width 0.2) (layer "B.Cu") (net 1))
 (segment (start 110.1725 105.450605) (end 113.521105 102.102) (width 0.2) (layer "B.Cu") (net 1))
 (segment (start 119.939895 99.978) (end 119.060105 99.978) (width 0.2) (layer "B.Cu") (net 1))
 (segment (start 120.562 100.600105) (end 119.939895 99.978) (width 0.2) (layer "B.Cu") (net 1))
 (segment (start 113.521105 102.102) (end 119.939895 102.102) (width 0.2) (layer "B.Cu") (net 1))
 (segment (start 120.562 101.479895) (end 120.562 100.600105) (width 0.2) (layer "B.Cu") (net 1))
 (segment (start 119.060105 99.978) (end 117.582105 98.5) (width 0.2) (layer "B.Cu") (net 1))
 (segment (start 110.1725 130.81) (end 110.1725 105.450605) (width 0.2) (layer "B.Cu") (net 1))
 (segment (start 72.0725 130.81) (end 99.3025 103.58) (width 0.2) (layer "B.Cu") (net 3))
 (segment (start 99.3025 103.58) (end 104.26 103.58) (width 0.2) (layer "B.Cu") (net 3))
 (segment (start 72.0725 130.81) (end 72.0725 149.86) (width 0.2) (layer "B.Cu") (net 3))
 (segment (start 125.351 134.269) (end 125.351 110.89337) (width 0.2) (layer "F.Cu") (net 11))
 (segment (start 120.57763 106.12) (end 119.5 106.12) (width 0.2) (layer "F.Cu") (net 11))
 (segment (start 123.5 136.12) (end 125.351 134.269) (width 0.2) (layer "F.Cu") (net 11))
 (segment (start 125.351 110.89337) (end 120.57763 106.12) (width 0.2) (layer "F.Cu") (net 11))
 (segment (start 85.5 136.12) (end 123.5 136.12) (width 0.2) (layer "F.Cu") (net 11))
 (segment (start 109.222 122.222365) (end 109.222 106.002) (width 0.2) (layer "B.Cu") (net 2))
 (segment (start 109.222 106.002) (end 104.26 101.04) (width 0.2) (layer "B.Cu") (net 2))
 (segment (start 100.634365 130.81) (end 109.222 122.222365) (width 0.2) (layer "B.Cu") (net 2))
 (segment (start 91.1225 130.81) (end 100.634365 130.81) (width 0.2) (layer "B.Cu") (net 2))
 (segment (start 91.1225 130.81) (end 91.1225 149.86) (width 0.2) (layer "B.Cu") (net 2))
 (segment (start 85.5 155.12) (end 104.5 155.12) (width 0.2) (layer "F.Cu") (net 10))
 (segment (start 121.590214 105.058) (end 119.060105 105.058) (width 0.2) (layer "F.Cu") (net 10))
 (segment (start 119.060105 105.058) (end 118.438 105.680105) (width 0.2) (layer "F.Cu") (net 10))
 (segment (start 126 110.976685) (end 125.751 110.727685) (width 0.2) (layer "F.Cu") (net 10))
 (segment (start 126 152.62) (end 126 110.976685) (width 0.2) (layer "F.Cu") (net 10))
 (segment (start 118.438 107.598) (end 119.5 108.66) (width 0.2) (layer "F.Cu") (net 10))
 (segment (start 123.5 155.12) (end 126 152.62) (width 0.2) (layer "F.Cu") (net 10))
 (segment (start 118.438 105.680105) (end 118.438 107.598) (width 0.2) (layer "F.Cu") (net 10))
 (segment (start 104.5 155.12) (end 123.5 155.12) (width 0.2) (layer "F.Cu") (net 10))
 (segment (start 125.751 110.727685) (end 125.751 109.218786) (width 0.2) (layer "F.Cu") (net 10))
 (segment (start 125.751 109.218786) (end 121.590214 105.058) (width 0.2) (layer "F.Cu") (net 10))
 (segment (start 85.27 128.27) (end 85.5 128.5) (width 0.2) (layer "F.Cu") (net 19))
 (segment (start 78.4225 128.27) (end 85.27 128.27) (width 0.2) (layer "F.Cu") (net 19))
 (segment (start 97.4725 128.27) (end 104.27 128.27) (width 0.2) (layer "F.Cu") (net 16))
 (segment (start 104.27 128.27) (end 104.5 128.5) (width 0.2) (layer "F.Cu") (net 16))
 (segment (start 123.27 128.27) (end 123.5 128.5) (width 0.2) (layer "F.Cu") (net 18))
 (segment (start 116.5225 128.27) (end 123.27 128.27) (width 0.2) (layer "F.Cu") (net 18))
 (segment (start 78.4225 147.32) (end 85.32 147.32) (width 0.2) (layer "F.Cu") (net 15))
 (segment (start 85.32 147.32) (end 85.5 147.5) (width 0.2) (layer "F.Cu") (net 15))
 (segment (start 104.32 147.32) (end 104.5 147.5) (width 0.2) (layer "F.Cu") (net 20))
 (segment (start 97.4725 147.32) (end 104.32 147.32) (width 0.2) (layer "F.Cu") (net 20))
 (segment (start 123.32 147.32) (end 123.5 147.5) (width 0.2) (layer "F.Cu") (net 17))
 (segment (start 116.5225 147.32) (end 123.32 147.32) (width 0.2) (layer "F.Cu") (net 17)))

